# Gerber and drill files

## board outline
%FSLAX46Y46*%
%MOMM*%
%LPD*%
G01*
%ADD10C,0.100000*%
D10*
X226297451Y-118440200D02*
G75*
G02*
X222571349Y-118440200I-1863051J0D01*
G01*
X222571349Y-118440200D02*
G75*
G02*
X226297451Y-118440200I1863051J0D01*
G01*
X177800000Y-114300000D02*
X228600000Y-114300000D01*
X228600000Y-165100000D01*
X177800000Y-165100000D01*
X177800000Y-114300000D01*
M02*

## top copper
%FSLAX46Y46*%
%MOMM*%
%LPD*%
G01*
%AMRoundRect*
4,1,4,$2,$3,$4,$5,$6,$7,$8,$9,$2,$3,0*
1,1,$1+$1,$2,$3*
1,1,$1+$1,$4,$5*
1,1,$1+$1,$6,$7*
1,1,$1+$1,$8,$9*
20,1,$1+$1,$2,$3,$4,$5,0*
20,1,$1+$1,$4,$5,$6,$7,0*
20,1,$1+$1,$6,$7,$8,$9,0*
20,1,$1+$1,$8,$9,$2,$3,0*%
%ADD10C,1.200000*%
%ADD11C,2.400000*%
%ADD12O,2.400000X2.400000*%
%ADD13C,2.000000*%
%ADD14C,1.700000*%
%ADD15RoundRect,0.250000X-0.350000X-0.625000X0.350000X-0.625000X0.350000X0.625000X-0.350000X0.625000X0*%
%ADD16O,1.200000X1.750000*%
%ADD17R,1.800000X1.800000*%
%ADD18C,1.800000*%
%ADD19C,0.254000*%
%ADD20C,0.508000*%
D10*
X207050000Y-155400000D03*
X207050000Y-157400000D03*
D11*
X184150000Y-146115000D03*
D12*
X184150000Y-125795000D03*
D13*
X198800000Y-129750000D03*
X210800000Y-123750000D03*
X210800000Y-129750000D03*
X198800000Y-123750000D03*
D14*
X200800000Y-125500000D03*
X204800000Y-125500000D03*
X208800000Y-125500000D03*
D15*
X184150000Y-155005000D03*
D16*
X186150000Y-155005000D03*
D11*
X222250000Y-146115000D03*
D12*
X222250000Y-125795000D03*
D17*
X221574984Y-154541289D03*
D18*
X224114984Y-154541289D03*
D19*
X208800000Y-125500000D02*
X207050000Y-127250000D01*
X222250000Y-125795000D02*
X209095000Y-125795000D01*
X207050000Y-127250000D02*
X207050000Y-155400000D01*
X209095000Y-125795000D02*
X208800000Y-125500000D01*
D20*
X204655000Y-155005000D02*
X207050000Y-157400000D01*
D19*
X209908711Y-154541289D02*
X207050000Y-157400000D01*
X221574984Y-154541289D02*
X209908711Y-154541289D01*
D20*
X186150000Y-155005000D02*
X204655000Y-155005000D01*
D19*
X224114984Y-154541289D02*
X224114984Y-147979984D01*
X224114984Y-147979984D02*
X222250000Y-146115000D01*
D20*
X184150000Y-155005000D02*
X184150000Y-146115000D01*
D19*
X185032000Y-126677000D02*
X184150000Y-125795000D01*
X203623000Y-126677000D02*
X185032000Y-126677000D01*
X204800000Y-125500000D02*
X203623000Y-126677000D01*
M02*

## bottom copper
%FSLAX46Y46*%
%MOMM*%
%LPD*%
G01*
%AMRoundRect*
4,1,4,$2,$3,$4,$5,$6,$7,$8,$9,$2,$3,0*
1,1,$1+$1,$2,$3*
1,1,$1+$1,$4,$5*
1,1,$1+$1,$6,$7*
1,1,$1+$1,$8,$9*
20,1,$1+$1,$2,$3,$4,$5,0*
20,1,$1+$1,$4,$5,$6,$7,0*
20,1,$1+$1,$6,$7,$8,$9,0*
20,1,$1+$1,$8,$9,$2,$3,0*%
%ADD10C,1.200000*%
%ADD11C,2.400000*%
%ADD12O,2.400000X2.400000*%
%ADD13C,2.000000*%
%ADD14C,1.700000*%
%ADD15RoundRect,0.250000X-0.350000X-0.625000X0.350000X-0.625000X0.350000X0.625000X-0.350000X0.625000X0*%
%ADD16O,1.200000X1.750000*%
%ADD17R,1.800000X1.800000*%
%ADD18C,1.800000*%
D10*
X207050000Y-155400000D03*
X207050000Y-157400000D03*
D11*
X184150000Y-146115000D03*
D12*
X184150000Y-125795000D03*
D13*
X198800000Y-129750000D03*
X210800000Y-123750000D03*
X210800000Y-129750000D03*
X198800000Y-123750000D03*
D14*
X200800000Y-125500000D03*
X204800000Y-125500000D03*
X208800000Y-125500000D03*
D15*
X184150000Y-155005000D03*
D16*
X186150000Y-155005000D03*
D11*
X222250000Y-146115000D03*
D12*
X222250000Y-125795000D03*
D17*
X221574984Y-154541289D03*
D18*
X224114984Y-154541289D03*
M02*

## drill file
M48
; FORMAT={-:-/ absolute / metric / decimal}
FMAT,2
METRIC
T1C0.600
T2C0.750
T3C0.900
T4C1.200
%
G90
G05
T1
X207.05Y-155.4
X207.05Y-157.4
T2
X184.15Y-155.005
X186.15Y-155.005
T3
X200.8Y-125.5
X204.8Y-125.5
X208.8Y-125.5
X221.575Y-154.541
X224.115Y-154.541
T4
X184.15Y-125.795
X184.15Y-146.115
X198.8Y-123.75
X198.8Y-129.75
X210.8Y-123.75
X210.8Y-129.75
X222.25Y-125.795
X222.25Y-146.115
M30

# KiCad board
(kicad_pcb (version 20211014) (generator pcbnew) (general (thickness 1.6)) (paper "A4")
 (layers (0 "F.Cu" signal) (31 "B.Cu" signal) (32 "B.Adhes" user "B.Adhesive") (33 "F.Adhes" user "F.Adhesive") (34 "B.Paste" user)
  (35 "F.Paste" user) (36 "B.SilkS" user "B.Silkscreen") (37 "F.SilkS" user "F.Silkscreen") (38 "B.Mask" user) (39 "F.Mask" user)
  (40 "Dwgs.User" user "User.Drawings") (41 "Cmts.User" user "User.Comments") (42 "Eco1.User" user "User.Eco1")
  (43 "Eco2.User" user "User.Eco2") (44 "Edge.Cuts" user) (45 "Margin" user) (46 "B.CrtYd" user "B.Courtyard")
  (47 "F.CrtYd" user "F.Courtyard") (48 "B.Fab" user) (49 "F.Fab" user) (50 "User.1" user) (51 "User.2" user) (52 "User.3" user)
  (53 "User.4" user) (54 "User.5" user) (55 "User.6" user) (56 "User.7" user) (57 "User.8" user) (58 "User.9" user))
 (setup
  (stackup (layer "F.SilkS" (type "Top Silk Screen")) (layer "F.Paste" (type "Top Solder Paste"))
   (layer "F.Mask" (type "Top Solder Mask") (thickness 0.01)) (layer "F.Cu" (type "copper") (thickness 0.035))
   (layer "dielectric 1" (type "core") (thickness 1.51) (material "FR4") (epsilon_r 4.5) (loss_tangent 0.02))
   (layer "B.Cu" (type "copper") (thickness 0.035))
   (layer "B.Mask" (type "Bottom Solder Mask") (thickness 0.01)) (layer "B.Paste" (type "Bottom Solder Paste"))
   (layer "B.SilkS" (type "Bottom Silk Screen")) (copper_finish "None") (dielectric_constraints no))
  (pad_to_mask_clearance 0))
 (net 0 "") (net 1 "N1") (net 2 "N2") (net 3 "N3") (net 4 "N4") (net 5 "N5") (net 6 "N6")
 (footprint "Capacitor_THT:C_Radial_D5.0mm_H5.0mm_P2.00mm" (layer "F.Cu") (at 207.05 155.4 -90)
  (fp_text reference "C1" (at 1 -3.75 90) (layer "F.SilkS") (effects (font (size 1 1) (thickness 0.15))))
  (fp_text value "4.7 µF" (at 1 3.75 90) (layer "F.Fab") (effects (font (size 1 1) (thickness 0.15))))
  (pad "1" thru_hole circle (at 0 0 270) (size 1.2 1.2) (drill 0.6) (layers *.Cu *.Mask) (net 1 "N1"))
  (pad "2" thru_hole circle (at 2 0 270) (size 1.2 1.2) (drill 0.6) (layers *.Cu *.Mask) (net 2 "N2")))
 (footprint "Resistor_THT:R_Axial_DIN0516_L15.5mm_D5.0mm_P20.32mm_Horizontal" (layer "F.Cu") (at 184.15 146.115 90)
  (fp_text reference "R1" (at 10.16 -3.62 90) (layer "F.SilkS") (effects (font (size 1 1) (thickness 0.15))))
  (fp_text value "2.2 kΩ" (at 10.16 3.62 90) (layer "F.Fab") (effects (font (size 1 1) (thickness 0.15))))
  (pad "1" thru_hole circle (at 0 0 90) (size 2.4 2.4) (drill 1.2) (layers *.Cu *.Mask) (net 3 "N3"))
  (pad "2" thru_hole oval (at 20.32 0 90) (size 2.4 2.4) (drill 1.2) (layers *.Cu *.Mask) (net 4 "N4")))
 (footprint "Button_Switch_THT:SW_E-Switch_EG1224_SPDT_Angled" (layer "F.Cu") (at 200.8 125.5)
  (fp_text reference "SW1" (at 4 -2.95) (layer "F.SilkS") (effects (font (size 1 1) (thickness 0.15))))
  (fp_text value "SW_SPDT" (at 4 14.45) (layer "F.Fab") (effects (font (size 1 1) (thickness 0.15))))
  (pad "" thru_hole circle (at -2 4.25) (size 2 2) (drill 1.2) (layers *.Cu *.Mask))
  (pad "" thru_hole circle (at 10 -1.75) (size 2 2) (drill 1.2) (layers *.Cu *.Mask))
  (pad "" thru_hole circle (at 10 4.25) (size 2 2) (drill 1.2) (layers *.Cu *.Mask))
  (pad "" thru_hole circle (at -2 -1.75) (size 2 2) (drill 1.2) (layers *.Cu *.Mask))
  (pad "1" thru_hole circle (at 0 0) (size 1.7 1.7) (drill 0.9) (layers *.Cu *.Mask) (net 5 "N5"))
  (pad "2" thru_hole circle (at 4 0) (size 1.7 1.7) (drill 0.9) (layers *.Cu *.Mask) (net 4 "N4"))
  (pad "3" thru_hole circle (at 8 0) (size 1.7 1.7) (drill 0.9) (layers *.Cu *.Mask) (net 1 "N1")))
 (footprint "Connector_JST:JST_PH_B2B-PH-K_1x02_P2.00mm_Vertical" (layer "F.Cu") (at 184.15 155.005)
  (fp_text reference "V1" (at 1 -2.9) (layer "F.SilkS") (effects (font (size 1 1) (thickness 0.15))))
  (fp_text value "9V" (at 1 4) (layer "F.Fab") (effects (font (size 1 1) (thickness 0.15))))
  (pad "1" thru_hole roundrect (at 0 0) (size 1.2 1.75) (drill 0.75) (layers *.Cu *.Mask) (roundrect_rratio 0.2083333333) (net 3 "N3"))
  (pad "2" thru_hole oval (at 2 0) (size 1.2 1.75) (drill 0.75) (layers *.Cu *.Mask) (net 2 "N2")))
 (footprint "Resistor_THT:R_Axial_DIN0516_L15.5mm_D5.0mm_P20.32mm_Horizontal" (layer "F.Cu") (at 222.25 146.115 90)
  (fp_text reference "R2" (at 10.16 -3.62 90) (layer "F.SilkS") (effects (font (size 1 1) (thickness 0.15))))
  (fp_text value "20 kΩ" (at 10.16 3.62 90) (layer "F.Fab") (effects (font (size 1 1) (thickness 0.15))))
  (pad "1" thru_hole circle (at 0 0 90) (size 2.4 2.4) (drill 1.2) (layers *.Cu *.Mask) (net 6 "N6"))
  (pad "2" thru_hole oval (at 20.32 0 90) (size 2.4 2.4) (drill 1.2) (layers *.Cu *.Mask) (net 1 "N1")))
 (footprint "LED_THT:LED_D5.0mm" (layer "F.Cu") (at 221.574984 154.541289)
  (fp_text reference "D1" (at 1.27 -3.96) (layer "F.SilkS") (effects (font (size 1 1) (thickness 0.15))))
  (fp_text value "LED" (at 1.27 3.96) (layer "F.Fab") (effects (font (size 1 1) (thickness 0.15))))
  (pad "1" thru_hole rect (at 0 0) (size 1.8 1.8) (drill 0.9) (layers *.Cu *.Mask) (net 2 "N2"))
  (pad "2" thru_hole circle (at 2.54 0) (size 1.8 1.8) (drill 0.9) (layers *.Cu *.Mask) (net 6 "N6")))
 (gr_circle (center 224.4344 118.4402) (end 226.1108 119.253) (layer "Edge.Cuts") (width 0.1) (fill none))
 (gr_rect (start 177.8 114.3) (end 228.6 165.1) (layer "Edge.Cuts") (width 0.1) (fill none))
 (segment (start 208.8 125.5) (end 207.05 127.25) (width 0.254) (layer "F.Cu") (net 1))
 (segment (start 222.25 125.795) (end 209.095 125.795) (width 0.254) (layer "F.Cu") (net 1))
 (segment (start 207.05 127.25) (end 207.05 155.4) (width 0.254) (layer "F.Cu") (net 1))
 (segment (start 209.095 125.795) (end 208.8 125.5) (width 0.254) (layer "F.Cu") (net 1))
 (segment (start 204.655 155.005) (end 207.05 157.4) (width 0.508) (layer "F.Cu") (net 2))
 (segment (start 209.908711 154.541289) (end 207.05 157.4) (width 0.254) (layer "F.Cu") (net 2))
 (segment (start 221.574984 154.541289) (end 209.908711 154.541289) (width 0.254) (layer "F.Cu") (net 2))
 (segment (start 186.15 155.005) (end 204.655 155.005) (width 0.508) (layer "F.Cu") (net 2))
 (segment (start 224.114984 154.541289) (end 224.114984 147.979984) (width 0.254) (layer "F.Cu") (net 6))
 (segment (start 224.114984 147.979984) (end 222.25 146.115) (width 0.254) (layer "F.Cu") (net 6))
 (segment (start 184.15 155.005) (end 184.15 146.115) (width 0.508) (layer "F.Cu") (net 3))
 (segment (start 185.032 126.677) (end 184.15 125.795) (width 0.254) (layer "F.Cu") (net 4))
 (segment (start 203.623 126.677) (end 185.032 126.677) (width 0.254) (layer "F.Cu") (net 4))
 (segment (start 204.8 125.5) (end 203.623 126.677) (width 0.254) (layer "F.Cu") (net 4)))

